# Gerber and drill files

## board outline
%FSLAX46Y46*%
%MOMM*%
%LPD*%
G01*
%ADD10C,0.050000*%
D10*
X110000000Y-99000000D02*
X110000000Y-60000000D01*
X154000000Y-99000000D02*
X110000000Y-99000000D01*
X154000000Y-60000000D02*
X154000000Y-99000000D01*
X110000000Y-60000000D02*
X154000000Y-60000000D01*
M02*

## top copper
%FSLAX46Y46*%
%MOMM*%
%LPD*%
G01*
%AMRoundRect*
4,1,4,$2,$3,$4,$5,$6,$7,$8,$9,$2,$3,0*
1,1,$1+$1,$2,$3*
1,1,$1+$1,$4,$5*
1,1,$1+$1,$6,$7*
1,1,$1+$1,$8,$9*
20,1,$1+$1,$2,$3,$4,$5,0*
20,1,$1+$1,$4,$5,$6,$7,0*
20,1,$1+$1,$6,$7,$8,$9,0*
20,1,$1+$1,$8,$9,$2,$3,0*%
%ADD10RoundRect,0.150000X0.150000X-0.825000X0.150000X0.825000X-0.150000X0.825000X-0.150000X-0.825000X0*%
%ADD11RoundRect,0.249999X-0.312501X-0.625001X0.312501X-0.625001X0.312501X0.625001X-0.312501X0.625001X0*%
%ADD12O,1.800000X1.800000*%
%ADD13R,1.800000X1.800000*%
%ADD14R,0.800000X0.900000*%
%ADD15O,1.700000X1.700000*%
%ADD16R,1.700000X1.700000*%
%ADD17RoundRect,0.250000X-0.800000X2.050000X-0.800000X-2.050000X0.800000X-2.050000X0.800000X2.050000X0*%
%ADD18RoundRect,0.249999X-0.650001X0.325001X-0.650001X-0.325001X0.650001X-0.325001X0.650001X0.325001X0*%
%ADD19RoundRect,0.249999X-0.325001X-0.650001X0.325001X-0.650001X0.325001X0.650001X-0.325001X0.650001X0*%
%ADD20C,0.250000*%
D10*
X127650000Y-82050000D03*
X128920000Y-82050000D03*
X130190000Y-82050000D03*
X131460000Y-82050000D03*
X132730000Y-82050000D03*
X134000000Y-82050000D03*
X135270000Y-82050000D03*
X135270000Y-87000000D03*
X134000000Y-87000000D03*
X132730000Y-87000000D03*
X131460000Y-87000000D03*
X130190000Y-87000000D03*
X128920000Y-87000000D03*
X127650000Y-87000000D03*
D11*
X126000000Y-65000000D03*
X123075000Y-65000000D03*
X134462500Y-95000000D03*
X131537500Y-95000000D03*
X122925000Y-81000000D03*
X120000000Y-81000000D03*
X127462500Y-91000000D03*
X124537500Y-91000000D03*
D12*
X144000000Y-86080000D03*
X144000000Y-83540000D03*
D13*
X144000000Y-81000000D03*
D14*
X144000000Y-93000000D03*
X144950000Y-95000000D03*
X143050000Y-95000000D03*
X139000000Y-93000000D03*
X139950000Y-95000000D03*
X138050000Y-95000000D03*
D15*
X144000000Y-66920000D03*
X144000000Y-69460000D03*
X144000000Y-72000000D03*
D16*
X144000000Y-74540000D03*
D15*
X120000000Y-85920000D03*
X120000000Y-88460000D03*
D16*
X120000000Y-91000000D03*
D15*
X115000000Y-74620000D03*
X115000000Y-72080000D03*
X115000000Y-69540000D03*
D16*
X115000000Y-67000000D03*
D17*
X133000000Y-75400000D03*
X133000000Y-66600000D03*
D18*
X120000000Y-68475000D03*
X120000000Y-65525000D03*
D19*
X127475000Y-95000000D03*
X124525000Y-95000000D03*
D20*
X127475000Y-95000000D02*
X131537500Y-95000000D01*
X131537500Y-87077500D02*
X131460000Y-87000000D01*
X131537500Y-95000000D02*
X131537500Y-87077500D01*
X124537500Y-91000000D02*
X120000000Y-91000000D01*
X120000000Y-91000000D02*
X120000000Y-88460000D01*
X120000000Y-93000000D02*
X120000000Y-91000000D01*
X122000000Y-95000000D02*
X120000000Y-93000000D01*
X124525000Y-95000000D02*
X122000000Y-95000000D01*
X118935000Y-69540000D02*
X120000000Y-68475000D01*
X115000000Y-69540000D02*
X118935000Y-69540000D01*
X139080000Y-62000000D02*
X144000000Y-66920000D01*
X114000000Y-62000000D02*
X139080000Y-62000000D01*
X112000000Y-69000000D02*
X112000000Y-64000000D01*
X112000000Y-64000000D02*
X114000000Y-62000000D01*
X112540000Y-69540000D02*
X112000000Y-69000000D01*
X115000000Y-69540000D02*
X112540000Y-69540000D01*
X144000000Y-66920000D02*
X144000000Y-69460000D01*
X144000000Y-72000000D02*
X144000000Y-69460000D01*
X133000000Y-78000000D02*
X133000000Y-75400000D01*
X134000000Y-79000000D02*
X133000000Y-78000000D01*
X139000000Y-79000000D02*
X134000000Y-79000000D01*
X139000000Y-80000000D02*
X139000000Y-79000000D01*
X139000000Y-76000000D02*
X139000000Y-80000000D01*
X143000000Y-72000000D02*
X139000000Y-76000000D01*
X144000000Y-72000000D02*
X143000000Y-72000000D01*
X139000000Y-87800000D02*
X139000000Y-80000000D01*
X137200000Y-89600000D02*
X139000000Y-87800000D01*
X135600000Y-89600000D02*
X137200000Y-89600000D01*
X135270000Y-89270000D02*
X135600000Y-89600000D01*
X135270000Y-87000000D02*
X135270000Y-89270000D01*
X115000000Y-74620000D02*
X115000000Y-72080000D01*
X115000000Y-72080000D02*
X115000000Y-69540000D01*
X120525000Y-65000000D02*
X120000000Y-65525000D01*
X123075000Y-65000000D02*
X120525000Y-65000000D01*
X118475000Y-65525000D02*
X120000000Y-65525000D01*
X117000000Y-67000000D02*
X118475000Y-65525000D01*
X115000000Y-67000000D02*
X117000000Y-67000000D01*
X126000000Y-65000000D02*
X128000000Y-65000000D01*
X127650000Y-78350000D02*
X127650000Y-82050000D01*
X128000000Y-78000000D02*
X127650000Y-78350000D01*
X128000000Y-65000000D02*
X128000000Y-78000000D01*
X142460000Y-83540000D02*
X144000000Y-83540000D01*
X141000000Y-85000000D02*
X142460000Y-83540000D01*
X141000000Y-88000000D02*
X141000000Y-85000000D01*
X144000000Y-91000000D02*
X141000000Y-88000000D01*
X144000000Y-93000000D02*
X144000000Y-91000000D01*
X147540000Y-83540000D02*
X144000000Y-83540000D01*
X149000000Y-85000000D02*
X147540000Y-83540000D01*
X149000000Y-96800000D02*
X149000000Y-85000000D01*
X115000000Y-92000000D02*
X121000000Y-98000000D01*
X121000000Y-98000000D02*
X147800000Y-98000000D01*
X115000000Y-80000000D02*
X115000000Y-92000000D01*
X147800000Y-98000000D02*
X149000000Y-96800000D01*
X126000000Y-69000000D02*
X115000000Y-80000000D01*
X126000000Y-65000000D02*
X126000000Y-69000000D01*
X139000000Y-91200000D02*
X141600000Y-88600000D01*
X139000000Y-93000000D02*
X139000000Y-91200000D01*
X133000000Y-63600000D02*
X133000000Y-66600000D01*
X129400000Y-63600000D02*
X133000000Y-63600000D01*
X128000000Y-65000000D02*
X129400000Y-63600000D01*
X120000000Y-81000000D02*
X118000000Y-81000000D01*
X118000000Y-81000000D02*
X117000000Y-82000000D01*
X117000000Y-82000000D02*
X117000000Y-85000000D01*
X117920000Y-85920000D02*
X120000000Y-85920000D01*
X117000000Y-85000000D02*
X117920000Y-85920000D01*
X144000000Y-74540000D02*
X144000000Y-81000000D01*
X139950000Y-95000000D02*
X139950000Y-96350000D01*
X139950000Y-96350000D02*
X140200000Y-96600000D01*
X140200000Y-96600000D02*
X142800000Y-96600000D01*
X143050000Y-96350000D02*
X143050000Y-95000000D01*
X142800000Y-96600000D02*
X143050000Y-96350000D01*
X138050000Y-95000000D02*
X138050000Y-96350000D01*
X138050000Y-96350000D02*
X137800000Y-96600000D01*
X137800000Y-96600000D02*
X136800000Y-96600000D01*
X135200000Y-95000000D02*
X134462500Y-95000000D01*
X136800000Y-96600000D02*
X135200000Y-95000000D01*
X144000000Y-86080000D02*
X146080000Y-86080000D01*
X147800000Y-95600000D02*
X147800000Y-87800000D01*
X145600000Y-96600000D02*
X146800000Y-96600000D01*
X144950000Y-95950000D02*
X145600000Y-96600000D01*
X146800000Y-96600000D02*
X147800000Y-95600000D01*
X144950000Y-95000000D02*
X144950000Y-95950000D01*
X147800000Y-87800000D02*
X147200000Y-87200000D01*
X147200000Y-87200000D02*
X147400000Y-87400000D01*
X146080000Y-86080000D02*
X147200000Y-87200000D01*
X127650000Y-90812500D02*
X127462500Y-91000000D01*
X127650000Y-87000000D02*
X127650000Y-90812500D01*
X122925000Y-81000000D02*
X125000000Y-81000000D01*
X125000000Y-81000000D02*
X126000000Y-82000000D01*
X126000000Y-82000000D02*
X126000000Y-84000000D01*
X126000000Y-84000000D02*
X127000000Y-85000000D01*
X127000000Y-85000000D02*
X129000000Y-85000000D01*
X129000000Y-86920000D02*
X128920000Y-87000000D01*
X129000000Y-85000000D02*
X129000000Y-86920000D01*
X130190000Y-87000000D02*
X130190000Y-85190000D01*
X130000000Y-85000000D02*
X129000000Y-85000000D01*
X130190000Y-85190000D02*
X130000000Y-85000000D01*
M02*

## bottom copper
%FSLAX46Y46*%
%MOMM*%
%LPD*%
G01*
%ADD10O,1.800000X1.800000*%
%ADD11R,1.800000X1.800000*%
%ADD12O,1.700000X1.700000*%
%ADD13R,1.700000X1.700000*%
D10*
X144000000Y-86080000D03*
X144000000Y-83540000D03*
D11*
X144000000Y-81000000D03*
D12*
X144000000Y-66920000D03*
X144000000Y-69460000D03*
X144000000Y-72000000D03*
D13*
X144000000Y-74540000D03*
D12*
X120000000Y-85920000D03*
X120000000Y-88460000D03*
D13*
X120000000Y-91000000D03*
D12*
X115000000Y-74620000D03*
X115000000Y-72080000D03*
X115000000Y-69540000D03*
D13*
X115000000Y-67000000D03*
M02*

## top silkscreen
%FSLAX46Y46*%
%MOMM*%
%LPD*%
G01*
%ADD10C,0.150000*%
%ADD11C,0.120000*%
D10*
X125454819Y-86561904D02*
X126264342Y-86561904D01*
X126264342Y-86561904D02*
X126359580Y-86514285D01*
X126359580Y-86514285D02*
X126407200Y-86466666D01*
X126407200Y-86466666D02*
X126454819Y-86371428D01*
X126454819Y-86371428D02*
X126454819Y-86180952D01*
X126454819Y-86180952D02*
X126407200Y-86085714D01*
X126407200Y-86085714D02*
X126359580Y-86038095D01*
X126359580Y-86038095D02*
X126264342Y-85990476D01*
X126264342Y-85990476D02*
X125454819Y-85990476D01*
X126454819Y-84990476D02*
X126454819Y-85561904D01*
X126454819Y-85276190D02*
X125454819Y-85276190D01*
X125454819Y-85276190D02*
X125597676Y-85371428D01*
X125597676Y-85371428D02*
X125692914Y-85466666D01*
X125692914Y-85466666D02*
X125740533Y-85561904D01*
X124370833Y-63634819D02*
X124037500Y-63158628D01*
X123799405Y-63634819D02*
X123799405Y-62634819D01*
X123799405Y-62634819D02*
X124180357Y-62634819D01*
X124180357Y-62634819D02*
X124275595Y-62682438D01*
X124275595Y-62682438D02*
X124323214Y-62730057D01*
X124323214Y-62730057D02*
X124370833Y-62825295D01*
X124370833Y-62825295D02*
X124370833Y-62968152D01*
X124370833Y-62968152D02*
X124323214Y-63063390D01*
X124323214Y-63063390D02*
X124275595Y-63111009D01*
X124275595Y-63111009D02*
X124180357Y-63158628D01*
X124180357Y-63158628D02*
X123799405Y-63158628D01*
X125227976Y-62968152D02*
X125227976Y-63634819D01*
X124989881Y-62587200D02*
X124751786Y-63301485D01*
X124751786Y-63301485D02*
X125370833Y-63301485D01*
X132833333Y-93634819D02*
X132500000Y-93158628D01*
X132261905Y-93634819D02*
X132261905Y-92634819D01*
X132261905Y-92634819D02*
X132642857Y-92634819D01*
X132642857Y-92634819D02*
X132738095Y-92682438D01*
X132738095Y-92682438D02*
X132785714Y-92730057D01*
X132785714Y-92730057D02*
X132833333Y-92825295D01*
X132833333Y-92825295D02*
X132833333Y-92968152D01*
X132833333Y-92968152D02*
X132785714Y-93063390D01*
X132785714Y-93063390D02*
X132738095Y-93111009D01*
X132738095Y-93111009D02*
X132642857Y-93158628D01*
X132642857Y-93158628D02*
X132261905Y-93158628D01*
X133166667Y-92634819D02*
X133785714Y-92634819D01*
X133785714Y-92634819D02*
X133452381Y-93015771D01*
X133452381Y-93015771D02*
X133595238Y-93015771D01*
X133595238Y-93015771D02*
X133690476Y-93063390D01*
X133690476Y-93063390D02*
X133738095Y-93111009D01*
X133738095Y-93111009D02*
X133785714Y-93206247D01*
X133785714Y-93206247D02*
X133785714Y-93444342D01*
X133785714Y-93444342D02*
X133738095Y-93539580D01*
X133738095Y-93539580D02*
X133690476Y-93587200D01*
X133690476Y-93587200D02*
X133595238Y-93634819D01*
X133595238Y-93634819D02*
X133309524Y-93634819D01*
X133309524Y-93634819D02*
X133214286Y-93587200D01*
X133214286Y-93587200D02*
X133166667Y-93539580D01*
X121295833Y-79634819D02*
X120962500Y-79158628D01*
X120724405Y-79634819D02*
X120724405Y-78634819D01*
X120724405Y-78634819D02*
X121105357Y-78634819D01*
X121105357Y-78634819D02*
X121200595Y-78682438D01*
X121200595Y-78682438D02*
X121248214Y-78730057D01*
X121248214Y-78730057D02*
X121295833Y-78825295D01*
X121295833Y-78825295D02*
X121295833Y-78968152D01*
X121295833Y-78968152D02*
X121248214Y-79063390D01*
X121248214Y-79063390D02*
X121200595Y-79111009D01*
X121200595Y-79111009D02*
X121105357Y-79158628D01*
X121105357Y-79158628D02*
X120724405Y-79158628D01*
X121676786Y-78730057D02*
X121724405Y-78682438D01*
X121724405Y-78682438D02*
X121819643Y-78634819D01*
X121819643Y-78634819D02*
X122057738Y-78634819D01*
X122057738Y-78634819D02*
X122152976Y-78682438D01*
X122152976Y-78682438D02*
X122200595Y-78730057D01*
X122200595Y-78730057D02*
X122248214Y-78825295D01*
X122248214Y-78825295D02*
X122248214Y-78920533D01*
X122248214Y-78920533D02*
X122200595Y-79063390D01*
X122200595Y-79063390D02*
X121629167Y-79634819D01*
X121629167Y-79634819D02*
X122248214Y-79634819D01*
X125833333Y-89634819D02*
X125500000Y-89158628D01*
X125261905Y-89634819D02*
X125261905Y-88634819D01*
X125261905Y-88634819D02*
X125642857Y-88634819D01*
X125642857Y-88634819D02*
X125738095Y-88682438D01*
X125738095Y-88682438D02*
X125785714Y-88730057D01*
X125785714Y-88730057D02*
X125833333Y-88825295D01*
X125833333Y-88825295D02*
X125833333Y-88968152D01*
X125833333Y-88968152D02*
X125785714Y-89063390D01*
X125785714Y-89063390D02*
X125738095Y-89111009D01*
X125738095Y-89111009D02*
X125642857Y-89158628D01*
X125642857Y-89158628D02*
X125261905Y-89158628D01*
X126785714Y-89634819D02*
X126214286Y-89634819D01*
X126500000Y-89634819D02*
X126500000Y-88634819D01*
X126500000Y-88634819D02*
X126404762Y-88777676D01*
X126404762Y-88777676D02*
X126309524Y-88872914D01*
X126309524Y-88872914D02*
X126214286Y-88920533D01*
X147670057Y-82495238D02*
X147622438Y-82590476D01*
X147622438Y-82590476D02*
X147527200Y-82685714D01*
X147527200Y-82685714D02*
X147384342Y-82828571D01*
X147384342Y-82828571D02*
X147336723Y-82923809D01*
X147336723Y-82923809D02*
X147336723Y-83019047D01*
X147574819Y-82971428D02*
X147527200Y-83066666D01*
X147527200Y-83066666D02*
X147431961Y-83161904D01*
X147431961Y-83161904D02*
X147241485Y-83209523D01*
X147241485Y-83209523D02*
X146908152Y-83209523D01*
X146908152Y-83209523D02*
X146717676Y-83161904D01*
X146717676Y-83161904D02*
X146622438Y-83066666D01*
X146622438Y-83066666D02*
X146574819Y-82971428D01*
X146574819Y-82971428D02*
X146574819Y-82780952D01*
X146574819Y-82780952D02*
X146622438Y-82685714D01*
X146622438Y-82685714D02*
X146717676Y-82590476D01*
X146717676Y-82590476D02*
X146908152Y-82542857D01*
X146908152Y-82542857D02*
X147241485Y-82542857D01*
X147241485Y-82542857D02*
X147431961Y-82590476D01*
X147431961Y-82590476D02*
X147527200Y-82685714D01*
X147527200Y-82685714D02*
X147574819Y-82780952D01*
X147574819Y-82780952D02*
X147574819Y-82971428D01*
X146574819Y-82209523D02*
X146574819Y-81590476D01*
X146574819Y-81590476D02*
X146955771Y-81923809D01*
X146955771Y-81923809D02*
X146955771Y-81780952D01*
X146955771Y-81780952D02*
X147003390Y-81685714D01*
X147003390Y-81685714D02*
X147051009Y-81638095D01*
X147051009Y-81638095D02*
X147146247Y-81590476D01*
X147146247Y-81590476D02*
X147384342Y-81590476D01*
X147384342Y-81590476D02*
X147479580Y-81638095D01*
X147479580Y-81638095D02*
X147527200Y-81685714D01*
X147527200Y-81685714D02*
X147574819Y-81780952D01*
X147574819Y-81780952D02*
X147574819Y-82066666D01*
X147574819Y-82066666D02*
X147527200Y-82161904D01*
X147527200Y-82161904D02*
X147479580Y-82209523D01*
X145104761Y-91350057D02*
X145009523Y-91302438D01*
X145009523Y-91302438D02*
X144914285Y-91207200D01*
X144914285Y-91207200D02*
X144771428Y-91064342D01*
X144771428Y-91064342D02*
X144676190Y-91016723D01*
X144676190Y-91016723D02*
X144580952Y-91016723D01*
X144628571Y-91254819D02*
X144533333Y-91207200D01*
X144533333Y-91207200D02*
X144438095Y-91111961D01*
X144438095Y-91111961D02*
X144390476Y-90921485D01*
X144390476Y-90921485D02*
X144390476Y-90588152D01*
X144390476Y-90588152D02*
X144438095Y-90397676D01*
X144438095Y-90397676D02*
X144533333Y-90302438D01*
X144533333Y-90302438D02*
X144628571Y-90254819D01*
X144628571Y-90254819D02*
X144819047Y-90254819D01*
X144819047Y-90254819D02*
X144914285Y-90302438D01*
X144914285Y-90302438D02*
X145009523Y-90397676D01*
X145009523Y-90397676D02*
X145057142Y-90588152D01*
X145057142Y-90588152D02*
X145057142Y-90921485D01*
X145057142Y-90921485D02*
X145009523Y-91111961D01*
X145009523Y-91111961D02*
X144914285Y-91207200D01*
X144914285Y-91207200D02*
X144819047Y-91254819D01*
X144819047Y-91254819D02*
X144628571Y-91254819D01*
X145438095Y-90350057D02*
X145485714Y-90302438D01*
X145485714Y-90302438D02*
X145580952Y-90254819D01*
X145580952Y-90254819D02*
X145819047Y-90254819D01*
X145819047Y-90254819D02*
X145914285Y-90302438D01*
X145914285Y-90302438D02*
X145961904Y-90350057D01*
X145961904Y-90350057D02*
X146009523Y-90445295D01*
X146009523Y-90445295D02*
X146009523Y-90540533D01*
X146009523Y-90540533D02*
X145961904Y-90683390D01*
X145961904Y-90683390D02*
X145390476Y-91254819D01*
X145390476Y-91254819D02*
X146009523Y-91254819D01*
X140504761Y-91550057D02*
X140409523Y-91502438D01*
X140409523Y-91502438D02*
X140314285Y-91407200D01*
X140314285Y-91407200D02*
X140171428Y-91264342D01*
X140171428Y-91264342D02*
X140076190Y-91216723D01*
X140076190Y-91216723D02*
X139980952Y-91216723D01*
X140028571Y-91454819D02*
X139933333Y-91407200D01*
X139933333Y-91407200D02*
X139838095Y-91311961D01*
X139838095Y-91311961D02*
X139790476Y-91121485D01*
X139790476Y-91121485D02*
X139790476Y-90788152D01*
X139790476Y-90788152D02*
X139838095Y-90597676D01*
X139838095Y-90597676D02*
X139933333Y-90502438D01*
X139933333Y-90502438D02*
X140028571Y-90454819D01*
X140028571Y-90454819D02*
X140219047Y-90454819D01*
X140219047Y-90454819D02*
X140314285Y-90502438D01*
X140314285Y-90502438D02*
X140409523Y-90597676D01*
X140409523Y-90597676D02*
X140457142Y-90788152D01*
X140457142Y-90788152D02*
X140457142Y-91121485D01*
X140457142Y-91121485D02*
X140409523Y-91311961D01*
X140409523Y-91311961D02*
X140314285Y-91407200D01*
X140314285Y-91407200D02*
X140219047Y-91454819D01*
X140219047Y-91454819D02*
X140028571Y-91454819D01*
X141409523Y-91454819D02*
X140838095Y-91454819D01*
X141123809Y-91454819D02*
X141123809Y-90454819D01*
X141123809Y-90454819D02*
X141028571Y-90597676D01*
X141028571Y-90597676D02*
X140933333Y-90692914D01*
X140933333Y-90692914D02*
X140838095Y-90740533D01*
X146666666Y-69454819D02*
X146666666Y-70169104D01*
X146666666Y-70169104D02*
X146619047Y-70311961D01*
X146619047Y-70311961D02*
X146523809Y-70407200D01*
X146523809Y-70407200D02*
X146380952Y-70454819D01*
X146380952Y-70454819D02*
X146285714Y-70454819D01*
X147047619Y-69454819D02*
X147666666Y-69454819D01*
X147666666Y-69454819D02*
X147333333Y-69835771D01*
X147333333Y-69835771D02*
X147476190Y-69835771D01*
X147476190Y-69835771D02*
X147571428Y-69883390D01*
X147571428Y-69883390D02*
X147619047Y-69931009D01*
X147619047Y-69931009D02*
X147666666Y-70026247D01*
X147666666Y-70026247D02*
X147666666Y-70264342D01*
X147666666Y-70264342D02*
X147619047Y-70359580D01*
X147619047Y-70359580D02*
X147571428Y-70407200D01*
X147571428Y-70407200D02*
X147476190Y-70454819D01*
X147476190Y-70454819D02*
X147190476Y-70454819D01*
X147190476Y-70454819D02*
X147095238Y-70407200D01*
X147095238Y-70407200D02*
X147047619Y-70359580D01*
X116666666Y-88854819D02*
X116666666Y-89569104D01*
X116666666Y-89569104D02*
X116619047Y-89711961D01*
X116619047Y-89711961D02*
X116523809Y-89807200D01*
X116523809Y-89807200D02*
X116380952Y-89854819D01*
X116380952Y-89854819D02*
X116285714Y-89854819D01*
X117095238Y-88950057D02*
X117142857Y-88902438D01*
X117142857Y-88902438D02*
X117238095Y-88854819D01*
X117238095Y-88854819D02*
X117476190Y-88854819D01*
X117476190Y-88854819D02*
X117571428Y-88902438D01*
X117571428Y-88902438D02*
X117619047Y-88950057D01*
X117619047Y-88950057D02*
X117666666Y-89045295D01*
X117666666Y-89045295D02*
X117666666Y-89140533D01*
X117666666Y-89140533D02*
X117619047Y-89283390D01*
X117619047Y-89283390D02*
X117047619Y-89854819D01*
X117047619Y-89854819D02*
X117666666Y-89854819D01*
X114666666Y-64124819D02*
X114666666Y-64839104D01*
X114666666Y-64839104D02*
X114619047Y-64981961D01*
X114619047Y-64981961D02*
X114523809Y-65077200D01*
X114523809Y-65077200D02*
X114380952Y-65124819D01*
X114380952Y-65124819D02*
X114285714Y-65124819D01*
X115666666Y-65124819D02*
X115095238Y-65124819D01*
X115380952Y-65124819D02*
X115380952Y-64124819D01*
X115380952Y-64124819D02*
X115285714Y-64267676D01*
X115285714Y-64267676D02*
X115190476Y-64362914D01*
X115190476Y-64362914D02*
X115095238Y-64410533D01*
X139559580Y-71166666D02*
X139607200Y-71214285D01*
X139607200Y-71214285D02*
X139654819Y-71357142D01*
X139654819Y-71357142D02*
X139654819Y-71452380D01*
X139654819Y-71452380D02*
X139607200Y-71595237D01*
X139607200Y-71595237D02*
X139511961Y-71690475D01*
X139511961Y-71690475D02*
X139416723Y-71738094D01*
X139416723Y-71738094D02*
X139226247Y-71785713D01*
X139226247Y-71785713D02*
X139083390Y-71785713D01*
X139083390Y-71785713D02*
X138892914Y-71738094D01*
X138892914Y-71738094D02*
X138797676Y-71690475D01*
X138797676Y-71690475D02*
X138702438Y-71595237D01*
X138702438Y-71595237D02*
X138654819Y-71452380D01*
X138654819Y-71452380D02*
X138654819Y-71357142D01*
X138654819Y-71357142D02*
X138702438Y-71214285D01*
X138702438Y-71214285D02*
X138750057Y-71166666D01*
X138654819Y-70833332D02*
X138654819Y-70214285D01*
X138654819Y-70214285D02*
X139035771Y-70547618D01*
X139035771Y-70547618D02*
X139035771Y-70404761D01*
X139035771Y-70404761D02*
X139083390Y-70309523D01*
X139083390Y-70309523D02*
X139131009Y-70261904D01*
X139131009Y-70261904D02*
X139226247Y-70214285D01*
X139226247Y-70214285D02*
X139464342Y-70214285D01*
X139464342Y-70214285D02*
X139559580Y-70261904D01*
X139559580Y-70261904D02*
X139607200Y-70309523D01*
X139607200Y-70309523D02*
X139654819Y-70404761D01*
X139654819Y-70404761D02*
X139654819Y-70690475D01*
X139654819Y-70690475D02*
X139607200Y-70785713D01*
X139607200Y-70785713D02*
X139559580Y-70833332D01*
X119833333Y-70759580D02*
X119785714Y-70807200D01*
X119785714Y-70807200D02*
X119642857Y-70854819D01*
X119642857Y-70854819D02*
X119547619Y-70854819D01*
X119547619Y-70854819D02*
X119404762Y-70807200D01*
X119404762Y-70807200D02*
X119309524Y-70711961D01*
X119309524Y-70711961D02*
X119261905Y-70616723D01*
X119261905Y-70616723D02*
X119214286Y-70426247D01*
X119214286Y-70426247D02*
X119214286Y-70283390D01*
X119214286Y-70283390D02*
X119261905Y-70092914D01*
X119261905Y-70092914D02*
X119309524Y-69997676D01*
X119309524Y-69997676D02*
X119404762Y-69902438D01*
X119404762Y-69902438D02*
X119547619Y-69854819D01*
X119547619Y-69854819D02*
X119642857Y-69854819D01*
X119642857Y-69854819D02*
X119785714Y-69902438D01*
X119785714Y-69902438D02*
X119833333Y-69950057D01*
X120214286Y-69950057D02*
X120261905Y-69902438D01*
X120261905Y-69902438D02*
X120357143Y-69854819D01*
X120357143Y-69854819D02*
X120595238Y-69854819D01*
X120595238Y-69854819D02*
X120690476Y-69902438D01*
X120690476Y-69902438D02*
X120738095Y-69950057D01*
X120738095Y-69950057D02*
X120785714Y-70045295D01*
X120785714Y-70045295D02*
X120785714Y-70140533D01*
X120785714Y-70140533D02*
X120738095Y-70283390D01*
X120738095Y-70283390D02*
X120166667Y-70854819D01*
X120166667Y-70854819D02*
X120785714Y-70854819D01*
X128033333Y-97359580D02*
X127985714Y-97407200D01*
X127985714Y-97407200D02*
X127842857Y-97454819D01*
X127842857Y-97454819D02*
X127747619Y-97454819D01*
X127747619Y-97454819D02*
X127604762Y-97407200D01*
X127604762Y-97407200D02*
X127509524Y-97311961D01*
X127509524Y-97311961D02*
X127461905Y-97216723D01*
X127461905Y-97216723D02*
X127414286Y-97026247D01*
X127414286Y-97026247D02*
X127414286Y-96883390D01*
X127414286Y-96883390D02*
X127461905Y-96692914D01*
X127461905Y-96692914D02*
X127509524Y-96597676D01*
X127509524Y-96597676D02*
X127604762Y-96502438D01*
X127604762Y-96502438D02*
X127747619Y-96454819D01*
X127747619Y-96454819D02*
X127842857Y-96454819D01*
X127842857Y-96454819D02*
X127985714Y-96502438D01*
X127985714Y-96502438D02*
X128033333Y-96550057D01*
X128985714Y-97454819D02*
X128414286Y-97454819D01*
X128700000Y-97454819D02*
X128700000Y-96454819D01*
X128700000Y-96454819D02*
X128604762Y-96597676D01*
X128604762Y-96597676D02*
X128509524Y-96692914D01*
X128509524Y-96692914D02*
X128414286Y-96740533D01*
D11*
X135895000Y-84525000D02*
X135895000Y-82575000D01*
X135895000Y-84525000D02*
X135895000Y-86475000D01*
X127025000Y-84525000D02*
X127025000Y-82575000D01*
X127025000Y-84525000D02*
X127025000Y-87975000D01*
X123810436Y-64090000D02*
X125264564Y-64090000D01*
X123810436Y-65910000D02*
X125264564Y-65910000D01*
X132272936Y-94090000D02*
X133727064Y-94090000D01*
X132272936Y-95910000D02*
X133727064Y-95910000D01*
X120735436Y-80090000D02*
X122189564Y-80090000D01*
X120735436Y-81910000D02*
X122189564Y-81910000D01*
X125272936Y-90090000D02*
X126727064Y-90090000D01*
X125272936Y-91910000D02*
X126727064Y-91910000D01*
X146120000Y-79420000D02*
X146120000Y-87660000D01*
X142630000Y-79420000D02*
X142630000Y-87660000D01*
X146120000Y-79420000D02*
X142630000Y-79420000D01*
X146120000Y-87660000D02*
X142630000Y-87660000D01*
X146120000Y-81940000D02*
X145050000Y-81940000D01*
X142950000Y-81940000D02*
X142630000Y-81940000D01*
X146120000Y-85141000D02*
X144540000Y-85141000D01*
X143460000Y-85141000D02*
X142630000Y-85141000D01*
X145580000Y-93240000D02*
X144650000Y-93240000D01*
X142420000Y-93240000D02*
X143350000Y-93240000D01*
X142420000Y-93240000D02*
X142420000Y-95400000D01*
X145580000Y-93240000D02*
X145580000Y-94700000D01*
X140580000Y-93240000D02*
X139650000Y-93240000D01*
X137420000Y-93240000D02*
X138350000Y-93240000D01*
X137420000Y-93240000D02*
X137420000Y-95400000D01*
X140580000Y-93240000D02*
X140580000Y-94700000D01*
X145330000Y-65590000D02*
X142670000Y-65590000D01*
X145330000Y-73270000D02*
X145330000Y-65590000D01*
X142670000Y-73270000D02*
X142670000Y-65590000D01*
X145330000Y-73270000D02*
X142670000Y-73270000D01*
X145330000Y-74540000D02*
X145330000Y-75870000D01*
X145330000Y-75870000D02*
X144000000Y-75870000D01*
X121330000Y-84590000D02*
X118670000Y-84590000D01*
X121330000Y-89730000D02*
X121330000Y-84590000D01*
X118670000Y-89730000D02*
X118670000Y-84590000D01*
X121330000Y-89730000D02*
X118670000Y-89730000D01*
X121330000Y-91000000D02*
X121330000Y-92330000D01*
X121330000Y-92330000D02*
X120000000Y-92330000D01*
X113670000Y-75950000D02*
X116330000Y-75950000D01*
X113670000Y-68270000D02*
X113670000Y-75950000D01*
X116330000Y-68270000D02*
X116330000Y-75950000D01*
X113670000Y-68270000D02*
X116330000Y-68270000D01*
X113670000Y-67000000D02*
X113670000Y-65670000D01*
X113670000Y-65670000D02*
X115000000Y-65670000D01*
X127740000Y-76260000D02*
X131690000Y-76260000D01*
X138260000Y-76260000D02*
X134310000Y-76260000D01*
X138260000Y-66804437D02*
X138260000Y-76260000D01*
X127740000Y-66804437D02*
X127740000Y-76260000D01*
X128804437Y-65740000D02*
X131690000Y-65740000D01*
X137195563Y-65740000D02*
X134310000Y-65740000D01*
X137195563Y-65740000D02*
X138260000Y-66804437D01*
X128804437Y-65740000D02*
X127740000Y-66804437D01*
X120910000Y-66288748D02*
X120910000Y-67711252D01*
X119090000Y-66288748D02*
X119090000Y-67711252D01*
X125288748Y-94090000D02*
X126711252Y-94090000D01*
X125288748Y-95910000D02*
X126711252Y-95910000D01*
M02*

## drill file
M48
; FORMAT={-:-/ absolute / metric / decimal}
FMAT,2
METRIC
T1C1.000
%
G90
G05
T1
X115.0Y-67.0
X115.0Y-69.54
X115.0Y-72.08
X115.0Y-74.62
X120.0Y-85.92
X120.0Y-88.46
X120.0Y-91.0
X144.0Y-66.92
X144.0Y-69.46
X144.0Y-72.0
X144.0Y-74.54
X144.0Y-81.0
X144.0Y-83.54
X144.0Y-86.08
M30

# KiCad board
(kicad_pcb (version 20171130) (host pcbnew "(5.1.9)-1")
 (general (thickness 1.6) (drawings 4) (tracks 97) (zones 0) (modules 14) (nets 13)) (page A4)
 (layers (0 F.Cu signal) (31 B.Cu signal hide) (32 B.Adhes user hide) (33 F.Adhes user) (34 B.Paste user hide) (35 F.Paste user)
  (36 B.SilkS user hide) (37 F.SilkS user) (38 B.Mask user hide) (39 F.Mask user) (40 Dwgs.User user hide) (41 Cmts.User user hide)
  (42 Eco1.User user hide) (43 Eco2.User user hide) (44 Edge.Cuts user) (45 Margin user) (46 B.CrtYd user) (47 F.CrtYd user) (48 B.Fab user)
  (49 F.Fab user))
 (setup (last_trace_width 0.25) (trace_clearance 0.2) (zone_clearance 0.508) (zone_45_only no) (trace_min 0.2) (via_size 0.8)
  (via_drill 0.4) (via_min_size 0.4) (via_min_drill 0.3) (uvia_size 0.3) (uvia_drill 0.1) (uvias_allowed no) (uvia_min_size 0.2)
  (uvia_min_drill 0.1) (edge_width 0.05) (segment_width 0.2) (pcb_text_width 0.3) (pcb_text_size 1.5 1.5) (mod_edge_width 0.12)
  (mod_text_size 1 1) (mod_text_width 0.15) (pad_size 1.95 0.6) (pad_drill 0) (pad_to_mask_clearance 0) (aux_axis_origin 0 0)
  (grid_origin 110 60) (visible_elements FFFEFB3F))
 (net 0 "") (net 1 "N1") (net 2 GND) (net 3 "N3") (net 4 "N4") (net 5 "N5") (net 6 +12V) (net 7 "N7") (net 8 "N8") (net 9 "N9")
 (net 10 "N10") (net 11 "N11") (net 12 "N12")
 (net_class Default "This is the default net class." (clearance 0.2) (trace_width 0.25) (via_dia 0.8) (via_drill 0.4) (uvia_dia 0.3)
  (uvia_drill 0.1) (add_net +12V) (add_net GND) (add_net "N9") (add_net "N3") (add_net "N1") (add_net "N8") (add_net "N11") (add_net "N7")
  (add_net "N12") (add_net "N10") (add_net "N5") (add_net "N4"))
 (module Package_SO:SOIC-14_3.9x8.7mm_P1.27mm (layer F.Cu) (at 131.46 84.525 90)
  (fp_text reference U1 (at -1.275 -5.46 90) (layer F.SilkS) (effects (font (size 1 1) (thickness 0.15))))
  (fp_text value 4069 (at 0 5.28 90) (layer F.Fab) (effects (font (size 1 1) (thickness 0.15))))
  (fp_line (start 0 4.435) (end 1.95 4.435) (layer F.SilkS) (width 0.12))
  (fp_line (start 0 4.435) (end -1.95 4.435) (layer F.SilkS) (width 0.12))
  (fp_line (start 0 -4.435) (end 1.95 -4.435) (layer F.SilkS) (width 0.12))
  (fp_line (start 0 -4.435) (end -3.45 -4.435) (layer F.SilkS) (width 0.12))
  (pad 14 smd roundrect (at 2.475 -3.81 90) (size 1.95 0.6) (layers F.Cu F.Paste F.Mask) (roundrect_rratio 0.25) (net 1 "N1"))
  (pad 13 smd roundrect (at 2.475 -2.54 90) (size 1.95 0.6) (layers F.Cu F.Paste F.Mask) (roundrect_rratio 0.25))
  (pad 12 smd roundrect (at 2.475 -1.27 90) (size 1.95 0.6) (layers F.Cu F.Paste F.Mask) (roundrect_rratio 0.25))
  (pad 11 smd roundrect (at 2.475 0 90) (size 1.95 0.6) (layers F.Cu F.Paste F.Mask) (roundrect_rratio 0.25))
  (pad 10 smd roundrect (at 2.475 1.27 90) (size 1.95 0.6) (layers F.Cu F.Paste F.Mask) (roundrect_rratio 0.25))
  (pad 9 smd roundrect (at 2.475 2.54 90) (size 1.95 0.6) (layers F.Cu F.Paste F.Mask) (roundrect_rratio 0.25))
  (pad 8 smd roundrect (at 2.475 3.81 90) (size 1.95 0.6) (layers F.Cu F.Paste F.Mask) (roundrect_rratio 0.25))
  (pad 7 smd roundrect (at -2.475 3.81 90) (size 1.95 0.6) (layers F.Cu F.Paste F.Mask) (roundrect_rratio 0.25) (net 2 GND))
  (pad 6 smd roundrect (at -2.475 2.54 90) (size 1.95 0.6) (layers F.Cu F.Paste F.Mask) (roundrect_rratio 0.25))
  (pad 5 smd roundrect (at -2.475 1.27 90) (size 1.95 0.6) (layers F.Cu F.Paste F.Mask) (roundrect_rratio 0.25))
  (pad 4 smd roundrect (at -2.475 0 90) (size 1.95 0.6) (layers F.Cu F.Paste F.Mask) (roundrect_rratio 0.25) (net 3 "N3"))
  (pad 3 smd roundrect (at -2.475 -1.27 90) (size 1.95 0.6) (layers F.Cu F.Paste F.Mask) (roundrect_rratio 0.25) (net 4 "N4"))
  (pad 2 smd roundrect (at -2.475 -2.54 90) (size 1.95 0.6) (layers F.Cu F.Paste F.Mask) (roundrect_rratio 0.25) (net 4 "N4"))
  (pad 1 smd roundrect (at -2.475 -3.81 90) (size 1.95 0.6) (layers F.Cu F.Paste F.Mask) (roundrect_rratio 0.25) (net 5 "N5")))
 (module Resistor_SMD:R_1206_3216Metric (layer F.Cu) (at 124.5375 65)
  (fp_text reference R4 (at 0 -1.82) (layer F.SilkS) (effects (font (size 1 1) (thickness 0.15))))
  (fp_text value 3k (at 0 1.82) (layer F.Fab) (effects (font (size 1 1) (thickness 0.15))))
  (fp_line (start -0.727064 -0.91) (end 0.727064 -0.91) (layer F.SilkS) (width 0.12))
  (fp_line (start -0.727064 0.91) (end 0.727064 0.91) (layer F.SilkS) (width 0.12))
  (pad 2 smd roundrect (at 1.4625 0) (size 1.125 1.75) (layers F.Cu F.Paste F.Mask) (roundrect_rratio 0.2222213333333333) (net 1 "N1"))
  (pad 1 smd roundrect (at -1.4625 0) (size 1.125 1.75) (layers F.Cu F.Paste F.Mask) (roundrect_rratio 0.2222213333333333) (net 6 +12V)))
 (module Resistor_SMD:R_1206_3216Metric (layer F.Cu) (at 133 95)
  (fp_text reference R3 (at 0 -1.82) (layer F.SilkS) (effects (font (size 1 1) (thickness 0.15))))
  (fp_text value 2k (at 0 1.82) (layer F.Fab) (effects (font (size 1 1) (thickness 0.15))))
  (fp_line (start -0.727064 -0.91) (end 0.727064 -0.91) (layer F.SilkS) (width 0.12))
  (fp_line (start -0.727064 0.91) (end 0.727064 0.91) (layer F.SilkS) (width 0.12))
  (pad 2 smd roundrect (at 1.4625 0) (size 1.125 1.75) (layers F.Cu F.Paste F.Mask) (roundrect_rratio 0.2222213333333333) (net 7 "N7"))
  (pad 1 smd roundrect (at -1.4625 0) (size 1.125 1.75) (layers F.Cu F.Paste F.Mask) (roundrect_rratio 0.2222213333333333) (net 3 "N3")))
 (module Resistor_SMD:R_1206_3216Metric (layer F.Cu) (at 121.4625 81)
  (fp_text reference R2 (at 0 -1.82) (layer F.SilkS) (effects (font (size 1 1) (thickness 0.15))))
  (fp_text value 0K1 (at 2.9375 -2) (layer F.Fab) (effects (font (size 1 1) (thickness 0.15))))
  (fp_line (start -0.727064 -0.91) (end 0.727064 -0.91) (layer F.SilkS) (width 0.12))
  (fp_line (start -0.727064 0.91) (end 0.727064 0.91) (layer F.SilkS) (width 0.12))
  (pad 2 smd roundrect (at 1.4625 0) (size 1.125 1.75) (layers F.Cu F.Paste F.Mask) (roundrect_rratio 0.2222213333333333) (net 4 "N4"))
  (pad 1 smd roundrect (at -1.4625 0) (size 1.125 1.75) (layers F.Cu F.Paste F.Mask) (roundrect_rratio 0.2222213333333333) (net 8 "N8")))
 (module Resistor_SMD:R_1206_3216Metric (layer F.Cu) (at 126 91)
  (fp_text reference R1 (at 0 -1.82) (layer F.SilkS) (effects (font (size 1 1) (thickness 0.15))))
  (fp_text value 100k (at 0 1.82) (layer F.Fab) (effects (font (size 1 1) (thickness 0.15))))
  (fp_line (start -0.727064 -0.91) (end 0.727064 -0.91) (layer F.SilkS) (width 0.12))
  (fp_line (start -0.727064 0.91) (end 0.727064 0.91) (layer F.SilkS) (width 0.12))
  (pad 2 smd roundrect (at 1.4625 0) (size 1.125 1.75) (layers F.Cu F.Paste F.Mask) (roundrect_rratio 0.2222213333333333) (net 5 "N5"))
  (pad 1 smd roundrect (at -1.4625 0) (size 1.125 1.75) (layers F.Cu F.Paste F.Mask) (roundrect_rratio 0.2222213333333333) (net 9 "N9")))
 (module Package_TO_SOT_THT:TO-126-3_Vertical (layer F.Cu) (at 144 81 270)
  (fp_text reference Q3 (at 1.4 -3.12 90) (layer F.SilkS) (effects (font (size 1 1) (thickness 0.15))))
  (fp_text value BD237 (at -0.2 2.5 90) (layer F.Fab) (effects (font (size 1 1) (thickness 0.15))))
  (fp_line (start -1.58 -2.12) (end 6.66 -2.12) (layer F.SilkS) (width 0.12))
  (fp_line (start -1.58 1.37) (end 6.66 1.37) (layer F.SilkS) (width 0.12))
  (fp_line (start -1.58 -2.12) (end -1.58 1.37) (layer F.SilkS) (width 0.12))
  (fp_line (start 6.66 -2.12) (end 6.66 1.37) (layer F.SilkS) (width 0.12))
  (fp_line (start 0.94 -2.12) (end 0.94 -1.05) (layer F.SilkS) (width 0.12))
  (fp_line (start 0.94 1.05) (end 0.94 1.37) (layer F.SilkS) (width 0.12))
  (fp_line (start 4.141 -2.12) (end 4.141 -0.54) (layer F.SilkS) (width 0.12))
  (fp_line (start 4.141 0.54) (end 4.141 1.37) (layer F.SilkS) (width 0.12))
  (pad 3 thru_hole oval (at 5.08 0 270) (size 1.8 1.8) (drill 1) (layers *.Cu *.Mask) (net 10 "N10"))
  (pad 2 thru_hole oval (at 2.54 0 270) (size 1.8 1.8) (drill 1) (layers *.Cu *.Mask) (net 1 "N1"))
  (pad 1 thru_hole rect (at 0 0 270) (size 1.8 1.8) (drill 1) (layers *.Cu *.Mask) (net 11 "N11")))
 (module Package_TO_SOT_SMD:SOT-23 (layer F.Cu) (at 144 94 90)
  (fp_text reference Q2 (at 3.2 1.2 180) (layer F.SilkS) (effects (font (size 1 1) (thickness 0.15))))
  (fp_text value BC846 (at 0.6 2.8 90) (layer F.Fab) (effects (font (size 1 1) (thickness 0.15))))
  (fp_line (start 0.76 1.58) (end 0.76 0.65) (layer F.SilkS) (width 0.12))
  (fp_line (start 0.76 -1.58) (end 0.76 -0.65) (layer F.SilkS) (width 0.12))
  (fp_line (start 0.76 -1.58) (end -1.4 -1.58) (layer F.SilkS) (width 0.12))
  (fp_line (start 0.76 1.58) (end -0.7 1.58) (layer F.SilkS) (width 0.12))
  (pad 3 smd rect (at 1 0 90) (size 0.9 0.8) (layers F.Cu F.Paste F.Mask) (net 1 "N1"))
  (pad 2 smd rect (at -1 0.95 90) (size 0.9 0.8) (layers F.Cu F.Paste F.Mask) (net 10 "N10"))
  (pad 1 smd rect (at -1 -0.95 90) (size 0.9 0.8) (layers F.Cu F.Paste F.Mask) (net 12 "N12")))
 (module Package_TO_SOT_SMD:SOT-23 (layer F.Cu) (at 139 94 90)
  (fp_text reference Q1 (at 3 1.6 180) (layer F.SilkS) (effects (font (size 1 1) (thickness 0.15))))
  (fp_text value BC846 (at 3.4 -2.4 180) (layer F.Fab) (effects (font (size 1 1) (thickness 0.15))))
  (fp_line (start 0.76 1.58) (end 0.76 0.65) (layer F.SilkS) (width 0.12))
  (fp_line (start 0.76 -1.58) (end 0.76 -0.65) (layer F.SilkS) (width 0.12))
  (fp_line (start 0.76 -1.58) (end -1.4 -1.58) (layer F.SilkS) (width 0.12))
  (fp_line (start 0.76 1.58) (end -0.7 1.58) (layer F.SilkS) (width 0.12))
  (pad 3 smd rect (at 1 0 90) (size 0.9 0.8) (layers F.Cu F.Paste F.Mask) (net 1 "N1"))
  (pad 2 smd rect (at -1 0.95 90) (size 0.9 0.8) (layers F.Cu F.Paste F.Mask) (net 12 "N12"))
  (pad 1 smd rect (at -1 -0.95 90) (size 0.9 0.8) (layers F.Cu F.Paste F.Mask) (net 7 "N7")))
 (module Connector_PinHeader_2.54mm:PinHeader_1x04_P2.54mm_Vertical (layer F.Cu) (at 144 74.54 180)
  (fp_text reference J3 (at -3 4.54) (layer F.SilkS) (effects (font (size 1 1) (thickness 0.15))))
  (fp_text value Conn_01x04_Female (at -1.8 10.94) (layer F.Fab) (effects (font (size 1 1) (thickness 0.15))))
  (fp_line (start -1.33 8.95) (end 1.33 8.95) (layer F.SilkS) (width 0.12))
  (fp_line (start -1.33 1.27) (end -1.33 8.95) (layer F.SilkS) (width 0.12))
  (fp_line (start 1.33 1.27) (end 1.33 8.95) (layer F.SilkS) (width 0.12))
  (fp_line (start -1.33 1.27) (end 1.33 1.27) (layer F.SilkS) (width 0.12))
  (fp_line (start -1.33 0) (end -1.33 -1.33) (layer F.SilkS) (width 0.12))
  (fp_line (start -1.33 -1.33) (end 0 -1.33) (layer F.SilkS) (width 0.12))
  (pad 4 thru_hole oval (at 0 7.62 180) (size 1.7 1.7) (drill 1) (layers *.Cu *.Mask) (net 2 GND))
  (pad 3 thru_hole oval (at 0 5.08 180) (size 1.7 1.7) (drill 1) (layers *.Cu *.Mask) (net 2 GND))
  (pad 2 thru_hole oval (at 0 2.54 180) (size 1.7 1.7) (drill 1) (layers *.Cu *.Mask) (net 2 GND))
  (pad 1 thru_hole rect (at 0 0 180) (size 1.7 1.7) (drill 1) (layers *.Cu *.Mask) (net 11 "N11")))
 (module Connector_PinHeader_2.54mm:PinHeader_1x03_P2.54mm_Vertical (layer F.Cu) (at 120 91 180)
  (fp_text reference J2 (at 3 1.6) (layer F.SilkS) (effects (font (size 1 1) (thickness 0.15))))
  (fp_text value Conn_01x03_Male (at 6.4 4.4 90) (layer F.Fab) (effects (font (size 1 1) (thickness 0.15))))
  (fp_line (start -1.33 6.41) (end 1.33 6.41) (layer F.SilkS) (width 0.12))
  (fp_line (start -1.33 1.27) (end -1.33 6.41) (layer F.SilkS) (width 0.12))
  (fp_line (start 1.33 1.27) (end 1.33 6.41) (layer F.SilkS) (width 0.12))
  (fp_line (start -1.33 1.27) (end 1.33 1.27) (layer F.SilkS) (width 0.12))
  (fp_line (start -1.33 0) (end -1.33 -1.33) (layer F.SilkS) (width 0.12))
  (fp_line (start -1.33 -1.33) (end 0 -1.33) (layer F.SilkS) (width 0.12))
  (pad 3 thru_hole oval (at 0 5.08 180) (size 1.7 1.7) (drill 1) (layers *.Cu *.Mask) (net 8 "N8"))
  (pad 2 thru_hole oval (at 0 2.54 180) (size 1.7 1.7) (drill 1) (layers *.Cu *.Mask) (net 9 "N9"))
  (pad 1 thru_hole rect (at 0 0 180) (size 1.7 1.7) (drill 1) (layers *.Cu *.Mask) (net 9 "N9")))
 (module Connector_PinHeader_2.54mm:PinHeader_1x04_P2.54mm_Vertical (layer F.Cu) (at 115 67)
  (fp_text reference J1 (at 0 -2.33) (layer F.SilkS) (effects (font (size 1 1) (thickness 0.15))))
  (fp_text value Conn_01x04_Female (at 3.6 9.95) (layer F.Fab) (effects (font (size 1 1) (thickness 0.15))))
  (fp_line (start -1.33 8.95) (end 1.33 8.95) (layer F.SilkS) (width 0.12))
  (fp_line (start -1.33 1.27) (end -1.33 8.95) (layer F.SilkS) (width 0.12))
  (fp_line (start 1.33 1.27) (end 1.33 8.95) (layer F.SilkS) (width 0.12))
  (fp_line (start -1.33 1.27) (end 1.33 1.27) (layer F.SilkS) (width 0.12))
  (fp_line (start -1.33 0) (end -1.33 -1.33) (layer F.SilkS) (width 0.12))
  (fp_line (start -1.33 -1.33) (end 0 -1.33) (layer F.SilkS) (width 0.12))
  (pad 4 thru_hole oval (at 0 7.62) (size 1.7 1.7) (drill 1) (layers *.Cu *.Mask) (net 2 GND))
  (pad 3 thru_hole oval (at 0 5.08) (size 1.7 1.7) (drill 1) (layers *.Cu *.Mask) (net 2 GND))
  (pad 2 thru_hole oval (at 0 2.54) (size 1.7 1.7) (drill 1) (layers *.Cu *.Mask) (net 2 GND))
  (pad 1 thru_hole rect (at 0 0) (size 1.7 1.7) (drill 1) (layers *.Cu *.Mask) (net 6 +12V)))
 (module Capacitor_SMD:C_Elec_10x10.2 (layer F.Cu) (at 133 71 270)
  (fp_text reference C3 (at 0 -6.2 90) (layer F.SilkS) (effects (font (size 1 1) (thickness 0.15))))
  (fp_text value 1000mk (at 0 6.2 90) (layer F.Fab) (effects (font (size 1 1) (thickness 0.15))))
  (fp_line (start 5.26 5.26) (end 5.26 1.31) (layer F.SilkS) (width 0.12))
  (fp_line (start 5.26 -5.26) (end 5.26 -1.31) (layer F.SilkS) (width 0.12))
  (fp_line (start -4.195563 -5.26) (end 5.26 -5.26) (layer F.SilkS) (width 0.12))
  (fp_line (start -4.195563 5.26) (end 5.26 5.26) (layer F.SilkS) (width 0.12))
  (fp_line (start -5.26 4.195563) (end -5.26 1.31) (layer F.SilkS) (width 0.12))
  (fp_line (start -5.26 -4.195563) (end -5.26 -1.31) (layer F.SilkS) (width 0.12))
  (fp_line (start -5.26 -4.195563) (end -4.195563 -5.26) (layer F.SilkS) (width 0.12))
  (fp_line (start -5.26 4.195563) (end -4.195563 5.26) (layer F.SilkS) (width 0.12))
  (pad 2 smd roundrect (at 4.4 0 270) (size 4.6 2.1) (layers F.Cu F.Paste F.Mask) (roundrect_rratio 0.119047619047619) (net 2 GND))
  (pad 1 smd roundrect (at -4.4 0 270) (size 4.6 2.1) (layers F.Cu F.Paste F.Mask) (roundrect_rratio 0.119047619047619) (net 1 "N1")))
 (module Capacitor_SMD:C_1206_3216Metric (layer F.Cu) (at 120 67 270)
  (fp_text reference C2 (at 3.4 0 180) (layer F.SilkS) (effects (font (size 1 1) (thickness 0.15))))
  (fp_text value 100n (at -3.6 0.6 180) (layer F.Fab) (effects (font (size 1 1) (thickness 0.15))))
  (fp_line (start -0.711252 -0.91) (end 0.711252 -0.91) (layer F.SilkS) (width 0.12))
  (fp_line (start -0.711252 0.91) (end 0.711252 0.91) (layer F.SilkS) (width 0.12))
  (pad 2 smd roundrect (at 1.475 0 270) (size 1.15 1.8) (layers F.Cu F.Paste F.Mask) (roundrect_rratio 0.2173904347826087) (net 2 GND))
  (pad 1 smd roundrect (at -1.475 0 270) (size 1.15 1.8) (layers F.Cu F.Paste F.Mask) (roundrect_rratio 0.2173904347826087) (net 6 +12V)))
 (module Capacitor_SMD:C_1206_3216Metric (layer F.Cu) (at 126 95)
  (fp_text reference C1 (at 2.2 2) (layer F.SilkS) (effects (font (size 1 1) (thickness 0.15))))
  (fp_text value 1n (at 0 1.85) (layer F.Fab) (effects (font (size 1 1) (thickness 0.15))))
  (fp_line (start -0.711252 -0.91) (end 0.711252 -0.91) (layer F.SilkS) (width 0.12))
  (fp_line (start -0.711252 0.91) (end 0.711252 0.91) (layer F.SilkS) (width 0.12))
  (pad 2 smd roundrect (at 1.475 0) (size 1.15 1.8) (layers F.Cu F.Paste F.Mask) (roundrect_rratio 0.2173904347826087) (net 3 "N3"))
  (pad 1 smd roundrect (at -1.475 0) (size 1.15 1.8) (layers F.Cu F.Paste F.Mask) (roundrect_rratio 0.2173904347826087) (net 9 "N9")))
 (gr_line (start 110 99) (end 110 60) (layer Edge.Cuts) (width 0.05))
 (gr_line (start 154 99) (end 110 99) (layer Edge.Cuts) (width 0.05))
 (gr_line (start 154 60) (end 154 99) (layer Edge.Cuts) (width 0.05))
 (gr_line (start 110 60) (end 154 60) (layer Edge.Cuts) (width 0.05))
 (segment (start 127.475 95) (end 131.5375 95) (width 0.25) (layer F.Cu) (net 3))
 (segment (start 131.5375 87.0775) (end 131.46 87) (width 0.25) (layer F.Cu) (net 3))
 (segment (start 131.5375 95) (end 131.5375 87.0775) (width 0.25) (layer F.Cu) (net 3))
 (segment (start 124.5375 91) (end 120 91) (width 0.25) (layer F.Cu) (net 9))
 (segment (start 120 91) (end 120 88.46) (width 0.25) (layer F.Cu) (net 9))
 (segment (start 120 93) (end 120 91) (width 0.25) (layer F.Cu) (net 9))
 (segment (start 122 95) (end 120 93) (width 0.25) (layer F.Cu) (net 9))
 (segment (start 124.525 95) (end 122 95) (width 0.25) (layer F.Cu) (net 9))
 (segment (start 118.935 69.54) (end 120 68.475) (width 0.25) (layer F.Cu) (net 2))
 (segment (start 115 69.54) (end 118.935 69.54) (width 0.25) (layer F.Cu) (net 2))
 (segment (start 139.08 62) (end 144 66.92) (width 0.25) (layer F.Cu) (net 2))
 (segment (start 114 62) (end 139.08 62) (width 0.25) (layer F.Cu) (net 2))
 (segment (start 112 69) (end 112 64) (width 0.25) (layer F.Cu) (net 2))
 (segment (start 112 64) (end 114 62) (width 0.25) (layer F.Cu) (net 2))
 (segment (start 112.54 69.54) (end 112 69) (width 0.25) (layer F.Cu) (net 2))
 (segment (start 115 69.54) (end 112.54 69.54) (width 0.25) (layer F.Cu) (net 2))
 (segment (start 144 66.92) (end 144 69.46) (width 0.25) (layer F.Cu) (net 2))
 (segment (start 144 72) (end 144 69.46) (width 0.25) (layer F.Cu) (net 2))
 (segment (start 133 78) (end 133 75.4) (width 0.25) (layer F.Cu) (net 2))
 (segment (start 134 79) (end 133 78) (width 0.25) (layer F.Cu) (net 2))
 (segment (start 139 79) (end 134 79) (width 0.25) (layer F.Cu) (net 2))
 (segment (start 139 80) (end 139 79) (width 0.25) (layer F.Cu) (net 2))
 (segment (start 139 76) (end 139 80) (width 0.25) (layer F.Cu) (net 2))
 (segment (start 143 72) (end 139 76) (width 0.25) (layer F.Cu) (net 2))
 (segment (start 144 72) (end 143 72) (width 0.25) (layer F.Cu) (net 2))
 (segment (start 139 87.8) (end 139 80) (width 0.25) (layer F.Cu) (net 2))
 (segment (start 137.2 89.6) (end 139 87.8) (width 0.25) (layer F.Cu) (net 2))
 (segment (start 135.6 89.6) (end 137.2 89.6) (width 0.25) (layer F.Cu) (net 2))
 (segment (start 135.27 89.27) (end 135.6 89.6) (width 0.25) (layer F.Cu) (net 2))
 (segment (start 135.27 87) (end 135.27 89.27) (width 0.25) (layer F.Cu) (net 2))
 (segment (start 115 74.62) (end 115 72.08) (width 0.25) (layer F.Cu) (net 2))
 (segment (start 115 72.08) (end 115 69.54) (width 0.25) (layer F.Cu) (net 2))
 (segment (start 120.525 65) (end 120 65.525) (width 0.25) (layer F.Cu) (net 6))
 (segment (start 123.075 65) (end 120.525 65) (width 0.25) (layer F.Cu) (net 6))
 (segment (start 118.475 65.525) (end 120 65.525) (width 0.25) (layer F.Cu) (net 6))
 (segment (start 117 67) (end 118.475 65.525) (width 0.25) (layer F.Cu) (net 6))
 (segment (start 115 67) (end 117 67) (width 0.25) (layer F.Cu) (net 6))
 (segment (start 126 65) (end 128 65) (width 0.25) (layer F.Cu) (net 1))
 (segment (start 127.65 78.35) (end 127.65 82.05) (width 0.25) (layer F.Cu) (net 1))
 (segment (start 128 78) (end 127.65 78.35) (width 0.25) (layer F.Cu) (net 1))
 (segment (start 128 65) (end 128 78) (width 0.25) (layer F.Cu) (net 1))
 (segment (start 142.46 83.54) (end 144 83.54) (width 0.25) (layer F.Cu) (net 1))
 (segment (start 141 85) (end 142.46 83.54) (width 0.25) (layer F.Cu) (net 1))
 (segment (start 141 88) (end 141 85) (width 0.25) (layer F.Cu) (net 1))
 (segment (start 144 91) (end 141 88) (width 0.25) (layer F.Cu) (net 1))
 (segment (start 144 93) (end 144 91) (width 0.25) (layer F.Cu) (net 1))
 (segment (start 147.54 83.54) (end 144 83.54) (width 0.25) (layer F.Cu) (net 1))
 (segment (start 149 85) (end 147.54 83.54) (width 0.25) (layer F.Cu) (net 1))
 (segment (start 149 96.8) (end 149 85) (width 0.25) (layer F.Cu) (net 1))
 (segment (start 115 92) (end 121 98) (width 0.25) (layer F.Cu) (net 1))
 (segment (start 121 98) (end 147.8 98) (width 0.25) (layer F.Cu) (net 1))
 (segment (start 115 80) (end 115 92) (width 0.25) (layer F.Cu) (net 1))
 (segment (start 147.8 98) (end 149 96.8) (width 0.25) (layer F.Cu) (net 1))
 (segment (start 126 69) (end 115 80) (width 0.25) (layer F.Cu) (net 1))
 (segment (start 126 65) (end 126 69) (width 0.25) (layer F.Cu) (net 1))
 (segment (start 139 91.2) (end 141.6 88.6) (width 0.25) (layer F.Cu) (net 1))
 (segment (start 139 93) (end 139 91.2) (width 0.25) (layer F.Cu) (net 1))
 (segment (start 133 63.6) (end 133 66.6) (width 0.25) (layer F.Cu) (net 1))
 (segment (start 129.4 63.6) (end 133 63.6) (width 0.25) (layer F.Cu) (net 1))
 (segment (start 128 65) (end 129.4 63.6) (width 0.25) (layer F.Cu) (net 1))
 (segment (start 120 81) (end 118 81) (width 0.25) (layer F.Cu) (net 8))
 (segment (start 118 81) (end 117 82) (width 0.25) (layer F.Cu) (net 8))
 (segment (start 117 82) (end 117 85) (width 0.25) (layer F.Cu) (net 8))
 (segment (start 117.92 85.92) (end 120 85.92) (width 0.25) (layer F.Cu) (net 8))
 (segment (start 117 85) (end 117.92 85.92) (width 0.25) (layer F.Cu) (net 8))
 (segment (start 144 74.54) (end 144 81) (width 0.25) (layer F.Cu) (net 11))
 (segment (start 139.95 95) (end 139.95 96.35) (width 0.25) (layer F.Cu) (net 12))
 (segment (start 139.95 96.35) (end 140.2 96.6) (width 0.25) (layer F.Cu) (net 12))
 (segment (start 140.2 96.6) (end 142.8 96.6) (width 0.25) (layer F.Cu) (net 12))
 (segment (start 143.05 96.35) (end 143.05 95) (width 0.25) (layer F.Cu) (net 12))
 (segment (start 142.8 96.6) (end 143.05 96.35) (width 0.25) (layer F.Cu) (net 12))
 (segment (start 138.05 95) (end 138.05 96.35) (width 0.25) (layer F.Cu) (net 7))
 (segment (start 138.05 96.35) (end 137.8 96.6) (width 0.25) (layer F.Cu) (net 7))
 (segment (start 137.8 96.6) (end 136.8 96.6) (width 0.25) (layer F.Cu) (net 7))
 (segment (start 135.2 95) (end 134.4625 95) (width 0.25) (layer F.Cu) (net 7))
 (segment (start 136.8 96.6) (end 135.2 95) (width 0.25) (layer F.Cu) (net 7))
 (segment (start 144 86.08) (end 146.08 86.08) (width 0.25) (layer F.Cu) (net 10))
 (segment (start 147.8 95.6) (end 147.8 87.8) (width 0.25) (layer F.Cu) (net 10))
 (segment (start 145.6 96.6) (end 146.8 96.6) (width 0.25) (layer F.Cu) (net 10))
 (segment (start 144.95 95.95) (end 145.6 96.6) (width 0.25) (layer F.Cu) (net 10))
 (segment (start 146.8 96.6) (end 147.8 95.6) (width 0.25) (layer F.Cu) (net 10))
 (segment (start 144.95 95) (end 144.95 95.95) (width 0.25) (layer F.Cu) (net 10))
 (segment (start 147.8 87.8) (end 147.2 87.2) (width 0.25) (layer F.Cu) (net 10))
 (segment (start 147.2 87.2) (end 147.4 87.4) (width 0.25) (layer F.Cu) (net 10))
 (segment (start 146.08 86.08) (end 147.2 87.2) (width 0.25) (layer F.Cu) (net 10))
 (segment (start 127.65 90.8125) (end 127.4625 91) (width 0.25) (layer F.Cu) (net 5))
 (segment (start 127.65 87) (end 127.65 90.8125) (width 0.25) (layer F.Cu) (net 5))
 (segment (start 122.925 81) (end 125 81) (width 0.25) (layer F.Cu) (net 4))
 (segment (start 125 81) (end 126 82) (width 0.25) (layer F.Cu) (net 4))
 (segment (start 126 82) (end 126 84) (width 0.25) (layer F.Cu) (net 4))
 (segment (start 126 84) (end 127 85) (width 0.25) (layer F.Cu) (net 4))
 (segment (start 127 85) (end 129 85) (width 0.25) (layer F.Cu) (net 4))
 (segment (start 129 86.92) (end 128.92 87) (width 0.25) (layer F.Cu) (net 4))
 (segment (start 129 85) (end 129 86.92) (width 0.25) (layer F.Cu) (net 4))
 (segment (start 130.19 87) (end 130.19 85.19) (width 0.25) (layer F.Cu) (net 4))
 (segment (start 130 85) (end 129 85) (width 0.25) (layer F.Cu) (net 4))
 (segment (start 130.19 85.19) (end 130 85) (width 0.25) (layer F.Cu) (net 4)))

